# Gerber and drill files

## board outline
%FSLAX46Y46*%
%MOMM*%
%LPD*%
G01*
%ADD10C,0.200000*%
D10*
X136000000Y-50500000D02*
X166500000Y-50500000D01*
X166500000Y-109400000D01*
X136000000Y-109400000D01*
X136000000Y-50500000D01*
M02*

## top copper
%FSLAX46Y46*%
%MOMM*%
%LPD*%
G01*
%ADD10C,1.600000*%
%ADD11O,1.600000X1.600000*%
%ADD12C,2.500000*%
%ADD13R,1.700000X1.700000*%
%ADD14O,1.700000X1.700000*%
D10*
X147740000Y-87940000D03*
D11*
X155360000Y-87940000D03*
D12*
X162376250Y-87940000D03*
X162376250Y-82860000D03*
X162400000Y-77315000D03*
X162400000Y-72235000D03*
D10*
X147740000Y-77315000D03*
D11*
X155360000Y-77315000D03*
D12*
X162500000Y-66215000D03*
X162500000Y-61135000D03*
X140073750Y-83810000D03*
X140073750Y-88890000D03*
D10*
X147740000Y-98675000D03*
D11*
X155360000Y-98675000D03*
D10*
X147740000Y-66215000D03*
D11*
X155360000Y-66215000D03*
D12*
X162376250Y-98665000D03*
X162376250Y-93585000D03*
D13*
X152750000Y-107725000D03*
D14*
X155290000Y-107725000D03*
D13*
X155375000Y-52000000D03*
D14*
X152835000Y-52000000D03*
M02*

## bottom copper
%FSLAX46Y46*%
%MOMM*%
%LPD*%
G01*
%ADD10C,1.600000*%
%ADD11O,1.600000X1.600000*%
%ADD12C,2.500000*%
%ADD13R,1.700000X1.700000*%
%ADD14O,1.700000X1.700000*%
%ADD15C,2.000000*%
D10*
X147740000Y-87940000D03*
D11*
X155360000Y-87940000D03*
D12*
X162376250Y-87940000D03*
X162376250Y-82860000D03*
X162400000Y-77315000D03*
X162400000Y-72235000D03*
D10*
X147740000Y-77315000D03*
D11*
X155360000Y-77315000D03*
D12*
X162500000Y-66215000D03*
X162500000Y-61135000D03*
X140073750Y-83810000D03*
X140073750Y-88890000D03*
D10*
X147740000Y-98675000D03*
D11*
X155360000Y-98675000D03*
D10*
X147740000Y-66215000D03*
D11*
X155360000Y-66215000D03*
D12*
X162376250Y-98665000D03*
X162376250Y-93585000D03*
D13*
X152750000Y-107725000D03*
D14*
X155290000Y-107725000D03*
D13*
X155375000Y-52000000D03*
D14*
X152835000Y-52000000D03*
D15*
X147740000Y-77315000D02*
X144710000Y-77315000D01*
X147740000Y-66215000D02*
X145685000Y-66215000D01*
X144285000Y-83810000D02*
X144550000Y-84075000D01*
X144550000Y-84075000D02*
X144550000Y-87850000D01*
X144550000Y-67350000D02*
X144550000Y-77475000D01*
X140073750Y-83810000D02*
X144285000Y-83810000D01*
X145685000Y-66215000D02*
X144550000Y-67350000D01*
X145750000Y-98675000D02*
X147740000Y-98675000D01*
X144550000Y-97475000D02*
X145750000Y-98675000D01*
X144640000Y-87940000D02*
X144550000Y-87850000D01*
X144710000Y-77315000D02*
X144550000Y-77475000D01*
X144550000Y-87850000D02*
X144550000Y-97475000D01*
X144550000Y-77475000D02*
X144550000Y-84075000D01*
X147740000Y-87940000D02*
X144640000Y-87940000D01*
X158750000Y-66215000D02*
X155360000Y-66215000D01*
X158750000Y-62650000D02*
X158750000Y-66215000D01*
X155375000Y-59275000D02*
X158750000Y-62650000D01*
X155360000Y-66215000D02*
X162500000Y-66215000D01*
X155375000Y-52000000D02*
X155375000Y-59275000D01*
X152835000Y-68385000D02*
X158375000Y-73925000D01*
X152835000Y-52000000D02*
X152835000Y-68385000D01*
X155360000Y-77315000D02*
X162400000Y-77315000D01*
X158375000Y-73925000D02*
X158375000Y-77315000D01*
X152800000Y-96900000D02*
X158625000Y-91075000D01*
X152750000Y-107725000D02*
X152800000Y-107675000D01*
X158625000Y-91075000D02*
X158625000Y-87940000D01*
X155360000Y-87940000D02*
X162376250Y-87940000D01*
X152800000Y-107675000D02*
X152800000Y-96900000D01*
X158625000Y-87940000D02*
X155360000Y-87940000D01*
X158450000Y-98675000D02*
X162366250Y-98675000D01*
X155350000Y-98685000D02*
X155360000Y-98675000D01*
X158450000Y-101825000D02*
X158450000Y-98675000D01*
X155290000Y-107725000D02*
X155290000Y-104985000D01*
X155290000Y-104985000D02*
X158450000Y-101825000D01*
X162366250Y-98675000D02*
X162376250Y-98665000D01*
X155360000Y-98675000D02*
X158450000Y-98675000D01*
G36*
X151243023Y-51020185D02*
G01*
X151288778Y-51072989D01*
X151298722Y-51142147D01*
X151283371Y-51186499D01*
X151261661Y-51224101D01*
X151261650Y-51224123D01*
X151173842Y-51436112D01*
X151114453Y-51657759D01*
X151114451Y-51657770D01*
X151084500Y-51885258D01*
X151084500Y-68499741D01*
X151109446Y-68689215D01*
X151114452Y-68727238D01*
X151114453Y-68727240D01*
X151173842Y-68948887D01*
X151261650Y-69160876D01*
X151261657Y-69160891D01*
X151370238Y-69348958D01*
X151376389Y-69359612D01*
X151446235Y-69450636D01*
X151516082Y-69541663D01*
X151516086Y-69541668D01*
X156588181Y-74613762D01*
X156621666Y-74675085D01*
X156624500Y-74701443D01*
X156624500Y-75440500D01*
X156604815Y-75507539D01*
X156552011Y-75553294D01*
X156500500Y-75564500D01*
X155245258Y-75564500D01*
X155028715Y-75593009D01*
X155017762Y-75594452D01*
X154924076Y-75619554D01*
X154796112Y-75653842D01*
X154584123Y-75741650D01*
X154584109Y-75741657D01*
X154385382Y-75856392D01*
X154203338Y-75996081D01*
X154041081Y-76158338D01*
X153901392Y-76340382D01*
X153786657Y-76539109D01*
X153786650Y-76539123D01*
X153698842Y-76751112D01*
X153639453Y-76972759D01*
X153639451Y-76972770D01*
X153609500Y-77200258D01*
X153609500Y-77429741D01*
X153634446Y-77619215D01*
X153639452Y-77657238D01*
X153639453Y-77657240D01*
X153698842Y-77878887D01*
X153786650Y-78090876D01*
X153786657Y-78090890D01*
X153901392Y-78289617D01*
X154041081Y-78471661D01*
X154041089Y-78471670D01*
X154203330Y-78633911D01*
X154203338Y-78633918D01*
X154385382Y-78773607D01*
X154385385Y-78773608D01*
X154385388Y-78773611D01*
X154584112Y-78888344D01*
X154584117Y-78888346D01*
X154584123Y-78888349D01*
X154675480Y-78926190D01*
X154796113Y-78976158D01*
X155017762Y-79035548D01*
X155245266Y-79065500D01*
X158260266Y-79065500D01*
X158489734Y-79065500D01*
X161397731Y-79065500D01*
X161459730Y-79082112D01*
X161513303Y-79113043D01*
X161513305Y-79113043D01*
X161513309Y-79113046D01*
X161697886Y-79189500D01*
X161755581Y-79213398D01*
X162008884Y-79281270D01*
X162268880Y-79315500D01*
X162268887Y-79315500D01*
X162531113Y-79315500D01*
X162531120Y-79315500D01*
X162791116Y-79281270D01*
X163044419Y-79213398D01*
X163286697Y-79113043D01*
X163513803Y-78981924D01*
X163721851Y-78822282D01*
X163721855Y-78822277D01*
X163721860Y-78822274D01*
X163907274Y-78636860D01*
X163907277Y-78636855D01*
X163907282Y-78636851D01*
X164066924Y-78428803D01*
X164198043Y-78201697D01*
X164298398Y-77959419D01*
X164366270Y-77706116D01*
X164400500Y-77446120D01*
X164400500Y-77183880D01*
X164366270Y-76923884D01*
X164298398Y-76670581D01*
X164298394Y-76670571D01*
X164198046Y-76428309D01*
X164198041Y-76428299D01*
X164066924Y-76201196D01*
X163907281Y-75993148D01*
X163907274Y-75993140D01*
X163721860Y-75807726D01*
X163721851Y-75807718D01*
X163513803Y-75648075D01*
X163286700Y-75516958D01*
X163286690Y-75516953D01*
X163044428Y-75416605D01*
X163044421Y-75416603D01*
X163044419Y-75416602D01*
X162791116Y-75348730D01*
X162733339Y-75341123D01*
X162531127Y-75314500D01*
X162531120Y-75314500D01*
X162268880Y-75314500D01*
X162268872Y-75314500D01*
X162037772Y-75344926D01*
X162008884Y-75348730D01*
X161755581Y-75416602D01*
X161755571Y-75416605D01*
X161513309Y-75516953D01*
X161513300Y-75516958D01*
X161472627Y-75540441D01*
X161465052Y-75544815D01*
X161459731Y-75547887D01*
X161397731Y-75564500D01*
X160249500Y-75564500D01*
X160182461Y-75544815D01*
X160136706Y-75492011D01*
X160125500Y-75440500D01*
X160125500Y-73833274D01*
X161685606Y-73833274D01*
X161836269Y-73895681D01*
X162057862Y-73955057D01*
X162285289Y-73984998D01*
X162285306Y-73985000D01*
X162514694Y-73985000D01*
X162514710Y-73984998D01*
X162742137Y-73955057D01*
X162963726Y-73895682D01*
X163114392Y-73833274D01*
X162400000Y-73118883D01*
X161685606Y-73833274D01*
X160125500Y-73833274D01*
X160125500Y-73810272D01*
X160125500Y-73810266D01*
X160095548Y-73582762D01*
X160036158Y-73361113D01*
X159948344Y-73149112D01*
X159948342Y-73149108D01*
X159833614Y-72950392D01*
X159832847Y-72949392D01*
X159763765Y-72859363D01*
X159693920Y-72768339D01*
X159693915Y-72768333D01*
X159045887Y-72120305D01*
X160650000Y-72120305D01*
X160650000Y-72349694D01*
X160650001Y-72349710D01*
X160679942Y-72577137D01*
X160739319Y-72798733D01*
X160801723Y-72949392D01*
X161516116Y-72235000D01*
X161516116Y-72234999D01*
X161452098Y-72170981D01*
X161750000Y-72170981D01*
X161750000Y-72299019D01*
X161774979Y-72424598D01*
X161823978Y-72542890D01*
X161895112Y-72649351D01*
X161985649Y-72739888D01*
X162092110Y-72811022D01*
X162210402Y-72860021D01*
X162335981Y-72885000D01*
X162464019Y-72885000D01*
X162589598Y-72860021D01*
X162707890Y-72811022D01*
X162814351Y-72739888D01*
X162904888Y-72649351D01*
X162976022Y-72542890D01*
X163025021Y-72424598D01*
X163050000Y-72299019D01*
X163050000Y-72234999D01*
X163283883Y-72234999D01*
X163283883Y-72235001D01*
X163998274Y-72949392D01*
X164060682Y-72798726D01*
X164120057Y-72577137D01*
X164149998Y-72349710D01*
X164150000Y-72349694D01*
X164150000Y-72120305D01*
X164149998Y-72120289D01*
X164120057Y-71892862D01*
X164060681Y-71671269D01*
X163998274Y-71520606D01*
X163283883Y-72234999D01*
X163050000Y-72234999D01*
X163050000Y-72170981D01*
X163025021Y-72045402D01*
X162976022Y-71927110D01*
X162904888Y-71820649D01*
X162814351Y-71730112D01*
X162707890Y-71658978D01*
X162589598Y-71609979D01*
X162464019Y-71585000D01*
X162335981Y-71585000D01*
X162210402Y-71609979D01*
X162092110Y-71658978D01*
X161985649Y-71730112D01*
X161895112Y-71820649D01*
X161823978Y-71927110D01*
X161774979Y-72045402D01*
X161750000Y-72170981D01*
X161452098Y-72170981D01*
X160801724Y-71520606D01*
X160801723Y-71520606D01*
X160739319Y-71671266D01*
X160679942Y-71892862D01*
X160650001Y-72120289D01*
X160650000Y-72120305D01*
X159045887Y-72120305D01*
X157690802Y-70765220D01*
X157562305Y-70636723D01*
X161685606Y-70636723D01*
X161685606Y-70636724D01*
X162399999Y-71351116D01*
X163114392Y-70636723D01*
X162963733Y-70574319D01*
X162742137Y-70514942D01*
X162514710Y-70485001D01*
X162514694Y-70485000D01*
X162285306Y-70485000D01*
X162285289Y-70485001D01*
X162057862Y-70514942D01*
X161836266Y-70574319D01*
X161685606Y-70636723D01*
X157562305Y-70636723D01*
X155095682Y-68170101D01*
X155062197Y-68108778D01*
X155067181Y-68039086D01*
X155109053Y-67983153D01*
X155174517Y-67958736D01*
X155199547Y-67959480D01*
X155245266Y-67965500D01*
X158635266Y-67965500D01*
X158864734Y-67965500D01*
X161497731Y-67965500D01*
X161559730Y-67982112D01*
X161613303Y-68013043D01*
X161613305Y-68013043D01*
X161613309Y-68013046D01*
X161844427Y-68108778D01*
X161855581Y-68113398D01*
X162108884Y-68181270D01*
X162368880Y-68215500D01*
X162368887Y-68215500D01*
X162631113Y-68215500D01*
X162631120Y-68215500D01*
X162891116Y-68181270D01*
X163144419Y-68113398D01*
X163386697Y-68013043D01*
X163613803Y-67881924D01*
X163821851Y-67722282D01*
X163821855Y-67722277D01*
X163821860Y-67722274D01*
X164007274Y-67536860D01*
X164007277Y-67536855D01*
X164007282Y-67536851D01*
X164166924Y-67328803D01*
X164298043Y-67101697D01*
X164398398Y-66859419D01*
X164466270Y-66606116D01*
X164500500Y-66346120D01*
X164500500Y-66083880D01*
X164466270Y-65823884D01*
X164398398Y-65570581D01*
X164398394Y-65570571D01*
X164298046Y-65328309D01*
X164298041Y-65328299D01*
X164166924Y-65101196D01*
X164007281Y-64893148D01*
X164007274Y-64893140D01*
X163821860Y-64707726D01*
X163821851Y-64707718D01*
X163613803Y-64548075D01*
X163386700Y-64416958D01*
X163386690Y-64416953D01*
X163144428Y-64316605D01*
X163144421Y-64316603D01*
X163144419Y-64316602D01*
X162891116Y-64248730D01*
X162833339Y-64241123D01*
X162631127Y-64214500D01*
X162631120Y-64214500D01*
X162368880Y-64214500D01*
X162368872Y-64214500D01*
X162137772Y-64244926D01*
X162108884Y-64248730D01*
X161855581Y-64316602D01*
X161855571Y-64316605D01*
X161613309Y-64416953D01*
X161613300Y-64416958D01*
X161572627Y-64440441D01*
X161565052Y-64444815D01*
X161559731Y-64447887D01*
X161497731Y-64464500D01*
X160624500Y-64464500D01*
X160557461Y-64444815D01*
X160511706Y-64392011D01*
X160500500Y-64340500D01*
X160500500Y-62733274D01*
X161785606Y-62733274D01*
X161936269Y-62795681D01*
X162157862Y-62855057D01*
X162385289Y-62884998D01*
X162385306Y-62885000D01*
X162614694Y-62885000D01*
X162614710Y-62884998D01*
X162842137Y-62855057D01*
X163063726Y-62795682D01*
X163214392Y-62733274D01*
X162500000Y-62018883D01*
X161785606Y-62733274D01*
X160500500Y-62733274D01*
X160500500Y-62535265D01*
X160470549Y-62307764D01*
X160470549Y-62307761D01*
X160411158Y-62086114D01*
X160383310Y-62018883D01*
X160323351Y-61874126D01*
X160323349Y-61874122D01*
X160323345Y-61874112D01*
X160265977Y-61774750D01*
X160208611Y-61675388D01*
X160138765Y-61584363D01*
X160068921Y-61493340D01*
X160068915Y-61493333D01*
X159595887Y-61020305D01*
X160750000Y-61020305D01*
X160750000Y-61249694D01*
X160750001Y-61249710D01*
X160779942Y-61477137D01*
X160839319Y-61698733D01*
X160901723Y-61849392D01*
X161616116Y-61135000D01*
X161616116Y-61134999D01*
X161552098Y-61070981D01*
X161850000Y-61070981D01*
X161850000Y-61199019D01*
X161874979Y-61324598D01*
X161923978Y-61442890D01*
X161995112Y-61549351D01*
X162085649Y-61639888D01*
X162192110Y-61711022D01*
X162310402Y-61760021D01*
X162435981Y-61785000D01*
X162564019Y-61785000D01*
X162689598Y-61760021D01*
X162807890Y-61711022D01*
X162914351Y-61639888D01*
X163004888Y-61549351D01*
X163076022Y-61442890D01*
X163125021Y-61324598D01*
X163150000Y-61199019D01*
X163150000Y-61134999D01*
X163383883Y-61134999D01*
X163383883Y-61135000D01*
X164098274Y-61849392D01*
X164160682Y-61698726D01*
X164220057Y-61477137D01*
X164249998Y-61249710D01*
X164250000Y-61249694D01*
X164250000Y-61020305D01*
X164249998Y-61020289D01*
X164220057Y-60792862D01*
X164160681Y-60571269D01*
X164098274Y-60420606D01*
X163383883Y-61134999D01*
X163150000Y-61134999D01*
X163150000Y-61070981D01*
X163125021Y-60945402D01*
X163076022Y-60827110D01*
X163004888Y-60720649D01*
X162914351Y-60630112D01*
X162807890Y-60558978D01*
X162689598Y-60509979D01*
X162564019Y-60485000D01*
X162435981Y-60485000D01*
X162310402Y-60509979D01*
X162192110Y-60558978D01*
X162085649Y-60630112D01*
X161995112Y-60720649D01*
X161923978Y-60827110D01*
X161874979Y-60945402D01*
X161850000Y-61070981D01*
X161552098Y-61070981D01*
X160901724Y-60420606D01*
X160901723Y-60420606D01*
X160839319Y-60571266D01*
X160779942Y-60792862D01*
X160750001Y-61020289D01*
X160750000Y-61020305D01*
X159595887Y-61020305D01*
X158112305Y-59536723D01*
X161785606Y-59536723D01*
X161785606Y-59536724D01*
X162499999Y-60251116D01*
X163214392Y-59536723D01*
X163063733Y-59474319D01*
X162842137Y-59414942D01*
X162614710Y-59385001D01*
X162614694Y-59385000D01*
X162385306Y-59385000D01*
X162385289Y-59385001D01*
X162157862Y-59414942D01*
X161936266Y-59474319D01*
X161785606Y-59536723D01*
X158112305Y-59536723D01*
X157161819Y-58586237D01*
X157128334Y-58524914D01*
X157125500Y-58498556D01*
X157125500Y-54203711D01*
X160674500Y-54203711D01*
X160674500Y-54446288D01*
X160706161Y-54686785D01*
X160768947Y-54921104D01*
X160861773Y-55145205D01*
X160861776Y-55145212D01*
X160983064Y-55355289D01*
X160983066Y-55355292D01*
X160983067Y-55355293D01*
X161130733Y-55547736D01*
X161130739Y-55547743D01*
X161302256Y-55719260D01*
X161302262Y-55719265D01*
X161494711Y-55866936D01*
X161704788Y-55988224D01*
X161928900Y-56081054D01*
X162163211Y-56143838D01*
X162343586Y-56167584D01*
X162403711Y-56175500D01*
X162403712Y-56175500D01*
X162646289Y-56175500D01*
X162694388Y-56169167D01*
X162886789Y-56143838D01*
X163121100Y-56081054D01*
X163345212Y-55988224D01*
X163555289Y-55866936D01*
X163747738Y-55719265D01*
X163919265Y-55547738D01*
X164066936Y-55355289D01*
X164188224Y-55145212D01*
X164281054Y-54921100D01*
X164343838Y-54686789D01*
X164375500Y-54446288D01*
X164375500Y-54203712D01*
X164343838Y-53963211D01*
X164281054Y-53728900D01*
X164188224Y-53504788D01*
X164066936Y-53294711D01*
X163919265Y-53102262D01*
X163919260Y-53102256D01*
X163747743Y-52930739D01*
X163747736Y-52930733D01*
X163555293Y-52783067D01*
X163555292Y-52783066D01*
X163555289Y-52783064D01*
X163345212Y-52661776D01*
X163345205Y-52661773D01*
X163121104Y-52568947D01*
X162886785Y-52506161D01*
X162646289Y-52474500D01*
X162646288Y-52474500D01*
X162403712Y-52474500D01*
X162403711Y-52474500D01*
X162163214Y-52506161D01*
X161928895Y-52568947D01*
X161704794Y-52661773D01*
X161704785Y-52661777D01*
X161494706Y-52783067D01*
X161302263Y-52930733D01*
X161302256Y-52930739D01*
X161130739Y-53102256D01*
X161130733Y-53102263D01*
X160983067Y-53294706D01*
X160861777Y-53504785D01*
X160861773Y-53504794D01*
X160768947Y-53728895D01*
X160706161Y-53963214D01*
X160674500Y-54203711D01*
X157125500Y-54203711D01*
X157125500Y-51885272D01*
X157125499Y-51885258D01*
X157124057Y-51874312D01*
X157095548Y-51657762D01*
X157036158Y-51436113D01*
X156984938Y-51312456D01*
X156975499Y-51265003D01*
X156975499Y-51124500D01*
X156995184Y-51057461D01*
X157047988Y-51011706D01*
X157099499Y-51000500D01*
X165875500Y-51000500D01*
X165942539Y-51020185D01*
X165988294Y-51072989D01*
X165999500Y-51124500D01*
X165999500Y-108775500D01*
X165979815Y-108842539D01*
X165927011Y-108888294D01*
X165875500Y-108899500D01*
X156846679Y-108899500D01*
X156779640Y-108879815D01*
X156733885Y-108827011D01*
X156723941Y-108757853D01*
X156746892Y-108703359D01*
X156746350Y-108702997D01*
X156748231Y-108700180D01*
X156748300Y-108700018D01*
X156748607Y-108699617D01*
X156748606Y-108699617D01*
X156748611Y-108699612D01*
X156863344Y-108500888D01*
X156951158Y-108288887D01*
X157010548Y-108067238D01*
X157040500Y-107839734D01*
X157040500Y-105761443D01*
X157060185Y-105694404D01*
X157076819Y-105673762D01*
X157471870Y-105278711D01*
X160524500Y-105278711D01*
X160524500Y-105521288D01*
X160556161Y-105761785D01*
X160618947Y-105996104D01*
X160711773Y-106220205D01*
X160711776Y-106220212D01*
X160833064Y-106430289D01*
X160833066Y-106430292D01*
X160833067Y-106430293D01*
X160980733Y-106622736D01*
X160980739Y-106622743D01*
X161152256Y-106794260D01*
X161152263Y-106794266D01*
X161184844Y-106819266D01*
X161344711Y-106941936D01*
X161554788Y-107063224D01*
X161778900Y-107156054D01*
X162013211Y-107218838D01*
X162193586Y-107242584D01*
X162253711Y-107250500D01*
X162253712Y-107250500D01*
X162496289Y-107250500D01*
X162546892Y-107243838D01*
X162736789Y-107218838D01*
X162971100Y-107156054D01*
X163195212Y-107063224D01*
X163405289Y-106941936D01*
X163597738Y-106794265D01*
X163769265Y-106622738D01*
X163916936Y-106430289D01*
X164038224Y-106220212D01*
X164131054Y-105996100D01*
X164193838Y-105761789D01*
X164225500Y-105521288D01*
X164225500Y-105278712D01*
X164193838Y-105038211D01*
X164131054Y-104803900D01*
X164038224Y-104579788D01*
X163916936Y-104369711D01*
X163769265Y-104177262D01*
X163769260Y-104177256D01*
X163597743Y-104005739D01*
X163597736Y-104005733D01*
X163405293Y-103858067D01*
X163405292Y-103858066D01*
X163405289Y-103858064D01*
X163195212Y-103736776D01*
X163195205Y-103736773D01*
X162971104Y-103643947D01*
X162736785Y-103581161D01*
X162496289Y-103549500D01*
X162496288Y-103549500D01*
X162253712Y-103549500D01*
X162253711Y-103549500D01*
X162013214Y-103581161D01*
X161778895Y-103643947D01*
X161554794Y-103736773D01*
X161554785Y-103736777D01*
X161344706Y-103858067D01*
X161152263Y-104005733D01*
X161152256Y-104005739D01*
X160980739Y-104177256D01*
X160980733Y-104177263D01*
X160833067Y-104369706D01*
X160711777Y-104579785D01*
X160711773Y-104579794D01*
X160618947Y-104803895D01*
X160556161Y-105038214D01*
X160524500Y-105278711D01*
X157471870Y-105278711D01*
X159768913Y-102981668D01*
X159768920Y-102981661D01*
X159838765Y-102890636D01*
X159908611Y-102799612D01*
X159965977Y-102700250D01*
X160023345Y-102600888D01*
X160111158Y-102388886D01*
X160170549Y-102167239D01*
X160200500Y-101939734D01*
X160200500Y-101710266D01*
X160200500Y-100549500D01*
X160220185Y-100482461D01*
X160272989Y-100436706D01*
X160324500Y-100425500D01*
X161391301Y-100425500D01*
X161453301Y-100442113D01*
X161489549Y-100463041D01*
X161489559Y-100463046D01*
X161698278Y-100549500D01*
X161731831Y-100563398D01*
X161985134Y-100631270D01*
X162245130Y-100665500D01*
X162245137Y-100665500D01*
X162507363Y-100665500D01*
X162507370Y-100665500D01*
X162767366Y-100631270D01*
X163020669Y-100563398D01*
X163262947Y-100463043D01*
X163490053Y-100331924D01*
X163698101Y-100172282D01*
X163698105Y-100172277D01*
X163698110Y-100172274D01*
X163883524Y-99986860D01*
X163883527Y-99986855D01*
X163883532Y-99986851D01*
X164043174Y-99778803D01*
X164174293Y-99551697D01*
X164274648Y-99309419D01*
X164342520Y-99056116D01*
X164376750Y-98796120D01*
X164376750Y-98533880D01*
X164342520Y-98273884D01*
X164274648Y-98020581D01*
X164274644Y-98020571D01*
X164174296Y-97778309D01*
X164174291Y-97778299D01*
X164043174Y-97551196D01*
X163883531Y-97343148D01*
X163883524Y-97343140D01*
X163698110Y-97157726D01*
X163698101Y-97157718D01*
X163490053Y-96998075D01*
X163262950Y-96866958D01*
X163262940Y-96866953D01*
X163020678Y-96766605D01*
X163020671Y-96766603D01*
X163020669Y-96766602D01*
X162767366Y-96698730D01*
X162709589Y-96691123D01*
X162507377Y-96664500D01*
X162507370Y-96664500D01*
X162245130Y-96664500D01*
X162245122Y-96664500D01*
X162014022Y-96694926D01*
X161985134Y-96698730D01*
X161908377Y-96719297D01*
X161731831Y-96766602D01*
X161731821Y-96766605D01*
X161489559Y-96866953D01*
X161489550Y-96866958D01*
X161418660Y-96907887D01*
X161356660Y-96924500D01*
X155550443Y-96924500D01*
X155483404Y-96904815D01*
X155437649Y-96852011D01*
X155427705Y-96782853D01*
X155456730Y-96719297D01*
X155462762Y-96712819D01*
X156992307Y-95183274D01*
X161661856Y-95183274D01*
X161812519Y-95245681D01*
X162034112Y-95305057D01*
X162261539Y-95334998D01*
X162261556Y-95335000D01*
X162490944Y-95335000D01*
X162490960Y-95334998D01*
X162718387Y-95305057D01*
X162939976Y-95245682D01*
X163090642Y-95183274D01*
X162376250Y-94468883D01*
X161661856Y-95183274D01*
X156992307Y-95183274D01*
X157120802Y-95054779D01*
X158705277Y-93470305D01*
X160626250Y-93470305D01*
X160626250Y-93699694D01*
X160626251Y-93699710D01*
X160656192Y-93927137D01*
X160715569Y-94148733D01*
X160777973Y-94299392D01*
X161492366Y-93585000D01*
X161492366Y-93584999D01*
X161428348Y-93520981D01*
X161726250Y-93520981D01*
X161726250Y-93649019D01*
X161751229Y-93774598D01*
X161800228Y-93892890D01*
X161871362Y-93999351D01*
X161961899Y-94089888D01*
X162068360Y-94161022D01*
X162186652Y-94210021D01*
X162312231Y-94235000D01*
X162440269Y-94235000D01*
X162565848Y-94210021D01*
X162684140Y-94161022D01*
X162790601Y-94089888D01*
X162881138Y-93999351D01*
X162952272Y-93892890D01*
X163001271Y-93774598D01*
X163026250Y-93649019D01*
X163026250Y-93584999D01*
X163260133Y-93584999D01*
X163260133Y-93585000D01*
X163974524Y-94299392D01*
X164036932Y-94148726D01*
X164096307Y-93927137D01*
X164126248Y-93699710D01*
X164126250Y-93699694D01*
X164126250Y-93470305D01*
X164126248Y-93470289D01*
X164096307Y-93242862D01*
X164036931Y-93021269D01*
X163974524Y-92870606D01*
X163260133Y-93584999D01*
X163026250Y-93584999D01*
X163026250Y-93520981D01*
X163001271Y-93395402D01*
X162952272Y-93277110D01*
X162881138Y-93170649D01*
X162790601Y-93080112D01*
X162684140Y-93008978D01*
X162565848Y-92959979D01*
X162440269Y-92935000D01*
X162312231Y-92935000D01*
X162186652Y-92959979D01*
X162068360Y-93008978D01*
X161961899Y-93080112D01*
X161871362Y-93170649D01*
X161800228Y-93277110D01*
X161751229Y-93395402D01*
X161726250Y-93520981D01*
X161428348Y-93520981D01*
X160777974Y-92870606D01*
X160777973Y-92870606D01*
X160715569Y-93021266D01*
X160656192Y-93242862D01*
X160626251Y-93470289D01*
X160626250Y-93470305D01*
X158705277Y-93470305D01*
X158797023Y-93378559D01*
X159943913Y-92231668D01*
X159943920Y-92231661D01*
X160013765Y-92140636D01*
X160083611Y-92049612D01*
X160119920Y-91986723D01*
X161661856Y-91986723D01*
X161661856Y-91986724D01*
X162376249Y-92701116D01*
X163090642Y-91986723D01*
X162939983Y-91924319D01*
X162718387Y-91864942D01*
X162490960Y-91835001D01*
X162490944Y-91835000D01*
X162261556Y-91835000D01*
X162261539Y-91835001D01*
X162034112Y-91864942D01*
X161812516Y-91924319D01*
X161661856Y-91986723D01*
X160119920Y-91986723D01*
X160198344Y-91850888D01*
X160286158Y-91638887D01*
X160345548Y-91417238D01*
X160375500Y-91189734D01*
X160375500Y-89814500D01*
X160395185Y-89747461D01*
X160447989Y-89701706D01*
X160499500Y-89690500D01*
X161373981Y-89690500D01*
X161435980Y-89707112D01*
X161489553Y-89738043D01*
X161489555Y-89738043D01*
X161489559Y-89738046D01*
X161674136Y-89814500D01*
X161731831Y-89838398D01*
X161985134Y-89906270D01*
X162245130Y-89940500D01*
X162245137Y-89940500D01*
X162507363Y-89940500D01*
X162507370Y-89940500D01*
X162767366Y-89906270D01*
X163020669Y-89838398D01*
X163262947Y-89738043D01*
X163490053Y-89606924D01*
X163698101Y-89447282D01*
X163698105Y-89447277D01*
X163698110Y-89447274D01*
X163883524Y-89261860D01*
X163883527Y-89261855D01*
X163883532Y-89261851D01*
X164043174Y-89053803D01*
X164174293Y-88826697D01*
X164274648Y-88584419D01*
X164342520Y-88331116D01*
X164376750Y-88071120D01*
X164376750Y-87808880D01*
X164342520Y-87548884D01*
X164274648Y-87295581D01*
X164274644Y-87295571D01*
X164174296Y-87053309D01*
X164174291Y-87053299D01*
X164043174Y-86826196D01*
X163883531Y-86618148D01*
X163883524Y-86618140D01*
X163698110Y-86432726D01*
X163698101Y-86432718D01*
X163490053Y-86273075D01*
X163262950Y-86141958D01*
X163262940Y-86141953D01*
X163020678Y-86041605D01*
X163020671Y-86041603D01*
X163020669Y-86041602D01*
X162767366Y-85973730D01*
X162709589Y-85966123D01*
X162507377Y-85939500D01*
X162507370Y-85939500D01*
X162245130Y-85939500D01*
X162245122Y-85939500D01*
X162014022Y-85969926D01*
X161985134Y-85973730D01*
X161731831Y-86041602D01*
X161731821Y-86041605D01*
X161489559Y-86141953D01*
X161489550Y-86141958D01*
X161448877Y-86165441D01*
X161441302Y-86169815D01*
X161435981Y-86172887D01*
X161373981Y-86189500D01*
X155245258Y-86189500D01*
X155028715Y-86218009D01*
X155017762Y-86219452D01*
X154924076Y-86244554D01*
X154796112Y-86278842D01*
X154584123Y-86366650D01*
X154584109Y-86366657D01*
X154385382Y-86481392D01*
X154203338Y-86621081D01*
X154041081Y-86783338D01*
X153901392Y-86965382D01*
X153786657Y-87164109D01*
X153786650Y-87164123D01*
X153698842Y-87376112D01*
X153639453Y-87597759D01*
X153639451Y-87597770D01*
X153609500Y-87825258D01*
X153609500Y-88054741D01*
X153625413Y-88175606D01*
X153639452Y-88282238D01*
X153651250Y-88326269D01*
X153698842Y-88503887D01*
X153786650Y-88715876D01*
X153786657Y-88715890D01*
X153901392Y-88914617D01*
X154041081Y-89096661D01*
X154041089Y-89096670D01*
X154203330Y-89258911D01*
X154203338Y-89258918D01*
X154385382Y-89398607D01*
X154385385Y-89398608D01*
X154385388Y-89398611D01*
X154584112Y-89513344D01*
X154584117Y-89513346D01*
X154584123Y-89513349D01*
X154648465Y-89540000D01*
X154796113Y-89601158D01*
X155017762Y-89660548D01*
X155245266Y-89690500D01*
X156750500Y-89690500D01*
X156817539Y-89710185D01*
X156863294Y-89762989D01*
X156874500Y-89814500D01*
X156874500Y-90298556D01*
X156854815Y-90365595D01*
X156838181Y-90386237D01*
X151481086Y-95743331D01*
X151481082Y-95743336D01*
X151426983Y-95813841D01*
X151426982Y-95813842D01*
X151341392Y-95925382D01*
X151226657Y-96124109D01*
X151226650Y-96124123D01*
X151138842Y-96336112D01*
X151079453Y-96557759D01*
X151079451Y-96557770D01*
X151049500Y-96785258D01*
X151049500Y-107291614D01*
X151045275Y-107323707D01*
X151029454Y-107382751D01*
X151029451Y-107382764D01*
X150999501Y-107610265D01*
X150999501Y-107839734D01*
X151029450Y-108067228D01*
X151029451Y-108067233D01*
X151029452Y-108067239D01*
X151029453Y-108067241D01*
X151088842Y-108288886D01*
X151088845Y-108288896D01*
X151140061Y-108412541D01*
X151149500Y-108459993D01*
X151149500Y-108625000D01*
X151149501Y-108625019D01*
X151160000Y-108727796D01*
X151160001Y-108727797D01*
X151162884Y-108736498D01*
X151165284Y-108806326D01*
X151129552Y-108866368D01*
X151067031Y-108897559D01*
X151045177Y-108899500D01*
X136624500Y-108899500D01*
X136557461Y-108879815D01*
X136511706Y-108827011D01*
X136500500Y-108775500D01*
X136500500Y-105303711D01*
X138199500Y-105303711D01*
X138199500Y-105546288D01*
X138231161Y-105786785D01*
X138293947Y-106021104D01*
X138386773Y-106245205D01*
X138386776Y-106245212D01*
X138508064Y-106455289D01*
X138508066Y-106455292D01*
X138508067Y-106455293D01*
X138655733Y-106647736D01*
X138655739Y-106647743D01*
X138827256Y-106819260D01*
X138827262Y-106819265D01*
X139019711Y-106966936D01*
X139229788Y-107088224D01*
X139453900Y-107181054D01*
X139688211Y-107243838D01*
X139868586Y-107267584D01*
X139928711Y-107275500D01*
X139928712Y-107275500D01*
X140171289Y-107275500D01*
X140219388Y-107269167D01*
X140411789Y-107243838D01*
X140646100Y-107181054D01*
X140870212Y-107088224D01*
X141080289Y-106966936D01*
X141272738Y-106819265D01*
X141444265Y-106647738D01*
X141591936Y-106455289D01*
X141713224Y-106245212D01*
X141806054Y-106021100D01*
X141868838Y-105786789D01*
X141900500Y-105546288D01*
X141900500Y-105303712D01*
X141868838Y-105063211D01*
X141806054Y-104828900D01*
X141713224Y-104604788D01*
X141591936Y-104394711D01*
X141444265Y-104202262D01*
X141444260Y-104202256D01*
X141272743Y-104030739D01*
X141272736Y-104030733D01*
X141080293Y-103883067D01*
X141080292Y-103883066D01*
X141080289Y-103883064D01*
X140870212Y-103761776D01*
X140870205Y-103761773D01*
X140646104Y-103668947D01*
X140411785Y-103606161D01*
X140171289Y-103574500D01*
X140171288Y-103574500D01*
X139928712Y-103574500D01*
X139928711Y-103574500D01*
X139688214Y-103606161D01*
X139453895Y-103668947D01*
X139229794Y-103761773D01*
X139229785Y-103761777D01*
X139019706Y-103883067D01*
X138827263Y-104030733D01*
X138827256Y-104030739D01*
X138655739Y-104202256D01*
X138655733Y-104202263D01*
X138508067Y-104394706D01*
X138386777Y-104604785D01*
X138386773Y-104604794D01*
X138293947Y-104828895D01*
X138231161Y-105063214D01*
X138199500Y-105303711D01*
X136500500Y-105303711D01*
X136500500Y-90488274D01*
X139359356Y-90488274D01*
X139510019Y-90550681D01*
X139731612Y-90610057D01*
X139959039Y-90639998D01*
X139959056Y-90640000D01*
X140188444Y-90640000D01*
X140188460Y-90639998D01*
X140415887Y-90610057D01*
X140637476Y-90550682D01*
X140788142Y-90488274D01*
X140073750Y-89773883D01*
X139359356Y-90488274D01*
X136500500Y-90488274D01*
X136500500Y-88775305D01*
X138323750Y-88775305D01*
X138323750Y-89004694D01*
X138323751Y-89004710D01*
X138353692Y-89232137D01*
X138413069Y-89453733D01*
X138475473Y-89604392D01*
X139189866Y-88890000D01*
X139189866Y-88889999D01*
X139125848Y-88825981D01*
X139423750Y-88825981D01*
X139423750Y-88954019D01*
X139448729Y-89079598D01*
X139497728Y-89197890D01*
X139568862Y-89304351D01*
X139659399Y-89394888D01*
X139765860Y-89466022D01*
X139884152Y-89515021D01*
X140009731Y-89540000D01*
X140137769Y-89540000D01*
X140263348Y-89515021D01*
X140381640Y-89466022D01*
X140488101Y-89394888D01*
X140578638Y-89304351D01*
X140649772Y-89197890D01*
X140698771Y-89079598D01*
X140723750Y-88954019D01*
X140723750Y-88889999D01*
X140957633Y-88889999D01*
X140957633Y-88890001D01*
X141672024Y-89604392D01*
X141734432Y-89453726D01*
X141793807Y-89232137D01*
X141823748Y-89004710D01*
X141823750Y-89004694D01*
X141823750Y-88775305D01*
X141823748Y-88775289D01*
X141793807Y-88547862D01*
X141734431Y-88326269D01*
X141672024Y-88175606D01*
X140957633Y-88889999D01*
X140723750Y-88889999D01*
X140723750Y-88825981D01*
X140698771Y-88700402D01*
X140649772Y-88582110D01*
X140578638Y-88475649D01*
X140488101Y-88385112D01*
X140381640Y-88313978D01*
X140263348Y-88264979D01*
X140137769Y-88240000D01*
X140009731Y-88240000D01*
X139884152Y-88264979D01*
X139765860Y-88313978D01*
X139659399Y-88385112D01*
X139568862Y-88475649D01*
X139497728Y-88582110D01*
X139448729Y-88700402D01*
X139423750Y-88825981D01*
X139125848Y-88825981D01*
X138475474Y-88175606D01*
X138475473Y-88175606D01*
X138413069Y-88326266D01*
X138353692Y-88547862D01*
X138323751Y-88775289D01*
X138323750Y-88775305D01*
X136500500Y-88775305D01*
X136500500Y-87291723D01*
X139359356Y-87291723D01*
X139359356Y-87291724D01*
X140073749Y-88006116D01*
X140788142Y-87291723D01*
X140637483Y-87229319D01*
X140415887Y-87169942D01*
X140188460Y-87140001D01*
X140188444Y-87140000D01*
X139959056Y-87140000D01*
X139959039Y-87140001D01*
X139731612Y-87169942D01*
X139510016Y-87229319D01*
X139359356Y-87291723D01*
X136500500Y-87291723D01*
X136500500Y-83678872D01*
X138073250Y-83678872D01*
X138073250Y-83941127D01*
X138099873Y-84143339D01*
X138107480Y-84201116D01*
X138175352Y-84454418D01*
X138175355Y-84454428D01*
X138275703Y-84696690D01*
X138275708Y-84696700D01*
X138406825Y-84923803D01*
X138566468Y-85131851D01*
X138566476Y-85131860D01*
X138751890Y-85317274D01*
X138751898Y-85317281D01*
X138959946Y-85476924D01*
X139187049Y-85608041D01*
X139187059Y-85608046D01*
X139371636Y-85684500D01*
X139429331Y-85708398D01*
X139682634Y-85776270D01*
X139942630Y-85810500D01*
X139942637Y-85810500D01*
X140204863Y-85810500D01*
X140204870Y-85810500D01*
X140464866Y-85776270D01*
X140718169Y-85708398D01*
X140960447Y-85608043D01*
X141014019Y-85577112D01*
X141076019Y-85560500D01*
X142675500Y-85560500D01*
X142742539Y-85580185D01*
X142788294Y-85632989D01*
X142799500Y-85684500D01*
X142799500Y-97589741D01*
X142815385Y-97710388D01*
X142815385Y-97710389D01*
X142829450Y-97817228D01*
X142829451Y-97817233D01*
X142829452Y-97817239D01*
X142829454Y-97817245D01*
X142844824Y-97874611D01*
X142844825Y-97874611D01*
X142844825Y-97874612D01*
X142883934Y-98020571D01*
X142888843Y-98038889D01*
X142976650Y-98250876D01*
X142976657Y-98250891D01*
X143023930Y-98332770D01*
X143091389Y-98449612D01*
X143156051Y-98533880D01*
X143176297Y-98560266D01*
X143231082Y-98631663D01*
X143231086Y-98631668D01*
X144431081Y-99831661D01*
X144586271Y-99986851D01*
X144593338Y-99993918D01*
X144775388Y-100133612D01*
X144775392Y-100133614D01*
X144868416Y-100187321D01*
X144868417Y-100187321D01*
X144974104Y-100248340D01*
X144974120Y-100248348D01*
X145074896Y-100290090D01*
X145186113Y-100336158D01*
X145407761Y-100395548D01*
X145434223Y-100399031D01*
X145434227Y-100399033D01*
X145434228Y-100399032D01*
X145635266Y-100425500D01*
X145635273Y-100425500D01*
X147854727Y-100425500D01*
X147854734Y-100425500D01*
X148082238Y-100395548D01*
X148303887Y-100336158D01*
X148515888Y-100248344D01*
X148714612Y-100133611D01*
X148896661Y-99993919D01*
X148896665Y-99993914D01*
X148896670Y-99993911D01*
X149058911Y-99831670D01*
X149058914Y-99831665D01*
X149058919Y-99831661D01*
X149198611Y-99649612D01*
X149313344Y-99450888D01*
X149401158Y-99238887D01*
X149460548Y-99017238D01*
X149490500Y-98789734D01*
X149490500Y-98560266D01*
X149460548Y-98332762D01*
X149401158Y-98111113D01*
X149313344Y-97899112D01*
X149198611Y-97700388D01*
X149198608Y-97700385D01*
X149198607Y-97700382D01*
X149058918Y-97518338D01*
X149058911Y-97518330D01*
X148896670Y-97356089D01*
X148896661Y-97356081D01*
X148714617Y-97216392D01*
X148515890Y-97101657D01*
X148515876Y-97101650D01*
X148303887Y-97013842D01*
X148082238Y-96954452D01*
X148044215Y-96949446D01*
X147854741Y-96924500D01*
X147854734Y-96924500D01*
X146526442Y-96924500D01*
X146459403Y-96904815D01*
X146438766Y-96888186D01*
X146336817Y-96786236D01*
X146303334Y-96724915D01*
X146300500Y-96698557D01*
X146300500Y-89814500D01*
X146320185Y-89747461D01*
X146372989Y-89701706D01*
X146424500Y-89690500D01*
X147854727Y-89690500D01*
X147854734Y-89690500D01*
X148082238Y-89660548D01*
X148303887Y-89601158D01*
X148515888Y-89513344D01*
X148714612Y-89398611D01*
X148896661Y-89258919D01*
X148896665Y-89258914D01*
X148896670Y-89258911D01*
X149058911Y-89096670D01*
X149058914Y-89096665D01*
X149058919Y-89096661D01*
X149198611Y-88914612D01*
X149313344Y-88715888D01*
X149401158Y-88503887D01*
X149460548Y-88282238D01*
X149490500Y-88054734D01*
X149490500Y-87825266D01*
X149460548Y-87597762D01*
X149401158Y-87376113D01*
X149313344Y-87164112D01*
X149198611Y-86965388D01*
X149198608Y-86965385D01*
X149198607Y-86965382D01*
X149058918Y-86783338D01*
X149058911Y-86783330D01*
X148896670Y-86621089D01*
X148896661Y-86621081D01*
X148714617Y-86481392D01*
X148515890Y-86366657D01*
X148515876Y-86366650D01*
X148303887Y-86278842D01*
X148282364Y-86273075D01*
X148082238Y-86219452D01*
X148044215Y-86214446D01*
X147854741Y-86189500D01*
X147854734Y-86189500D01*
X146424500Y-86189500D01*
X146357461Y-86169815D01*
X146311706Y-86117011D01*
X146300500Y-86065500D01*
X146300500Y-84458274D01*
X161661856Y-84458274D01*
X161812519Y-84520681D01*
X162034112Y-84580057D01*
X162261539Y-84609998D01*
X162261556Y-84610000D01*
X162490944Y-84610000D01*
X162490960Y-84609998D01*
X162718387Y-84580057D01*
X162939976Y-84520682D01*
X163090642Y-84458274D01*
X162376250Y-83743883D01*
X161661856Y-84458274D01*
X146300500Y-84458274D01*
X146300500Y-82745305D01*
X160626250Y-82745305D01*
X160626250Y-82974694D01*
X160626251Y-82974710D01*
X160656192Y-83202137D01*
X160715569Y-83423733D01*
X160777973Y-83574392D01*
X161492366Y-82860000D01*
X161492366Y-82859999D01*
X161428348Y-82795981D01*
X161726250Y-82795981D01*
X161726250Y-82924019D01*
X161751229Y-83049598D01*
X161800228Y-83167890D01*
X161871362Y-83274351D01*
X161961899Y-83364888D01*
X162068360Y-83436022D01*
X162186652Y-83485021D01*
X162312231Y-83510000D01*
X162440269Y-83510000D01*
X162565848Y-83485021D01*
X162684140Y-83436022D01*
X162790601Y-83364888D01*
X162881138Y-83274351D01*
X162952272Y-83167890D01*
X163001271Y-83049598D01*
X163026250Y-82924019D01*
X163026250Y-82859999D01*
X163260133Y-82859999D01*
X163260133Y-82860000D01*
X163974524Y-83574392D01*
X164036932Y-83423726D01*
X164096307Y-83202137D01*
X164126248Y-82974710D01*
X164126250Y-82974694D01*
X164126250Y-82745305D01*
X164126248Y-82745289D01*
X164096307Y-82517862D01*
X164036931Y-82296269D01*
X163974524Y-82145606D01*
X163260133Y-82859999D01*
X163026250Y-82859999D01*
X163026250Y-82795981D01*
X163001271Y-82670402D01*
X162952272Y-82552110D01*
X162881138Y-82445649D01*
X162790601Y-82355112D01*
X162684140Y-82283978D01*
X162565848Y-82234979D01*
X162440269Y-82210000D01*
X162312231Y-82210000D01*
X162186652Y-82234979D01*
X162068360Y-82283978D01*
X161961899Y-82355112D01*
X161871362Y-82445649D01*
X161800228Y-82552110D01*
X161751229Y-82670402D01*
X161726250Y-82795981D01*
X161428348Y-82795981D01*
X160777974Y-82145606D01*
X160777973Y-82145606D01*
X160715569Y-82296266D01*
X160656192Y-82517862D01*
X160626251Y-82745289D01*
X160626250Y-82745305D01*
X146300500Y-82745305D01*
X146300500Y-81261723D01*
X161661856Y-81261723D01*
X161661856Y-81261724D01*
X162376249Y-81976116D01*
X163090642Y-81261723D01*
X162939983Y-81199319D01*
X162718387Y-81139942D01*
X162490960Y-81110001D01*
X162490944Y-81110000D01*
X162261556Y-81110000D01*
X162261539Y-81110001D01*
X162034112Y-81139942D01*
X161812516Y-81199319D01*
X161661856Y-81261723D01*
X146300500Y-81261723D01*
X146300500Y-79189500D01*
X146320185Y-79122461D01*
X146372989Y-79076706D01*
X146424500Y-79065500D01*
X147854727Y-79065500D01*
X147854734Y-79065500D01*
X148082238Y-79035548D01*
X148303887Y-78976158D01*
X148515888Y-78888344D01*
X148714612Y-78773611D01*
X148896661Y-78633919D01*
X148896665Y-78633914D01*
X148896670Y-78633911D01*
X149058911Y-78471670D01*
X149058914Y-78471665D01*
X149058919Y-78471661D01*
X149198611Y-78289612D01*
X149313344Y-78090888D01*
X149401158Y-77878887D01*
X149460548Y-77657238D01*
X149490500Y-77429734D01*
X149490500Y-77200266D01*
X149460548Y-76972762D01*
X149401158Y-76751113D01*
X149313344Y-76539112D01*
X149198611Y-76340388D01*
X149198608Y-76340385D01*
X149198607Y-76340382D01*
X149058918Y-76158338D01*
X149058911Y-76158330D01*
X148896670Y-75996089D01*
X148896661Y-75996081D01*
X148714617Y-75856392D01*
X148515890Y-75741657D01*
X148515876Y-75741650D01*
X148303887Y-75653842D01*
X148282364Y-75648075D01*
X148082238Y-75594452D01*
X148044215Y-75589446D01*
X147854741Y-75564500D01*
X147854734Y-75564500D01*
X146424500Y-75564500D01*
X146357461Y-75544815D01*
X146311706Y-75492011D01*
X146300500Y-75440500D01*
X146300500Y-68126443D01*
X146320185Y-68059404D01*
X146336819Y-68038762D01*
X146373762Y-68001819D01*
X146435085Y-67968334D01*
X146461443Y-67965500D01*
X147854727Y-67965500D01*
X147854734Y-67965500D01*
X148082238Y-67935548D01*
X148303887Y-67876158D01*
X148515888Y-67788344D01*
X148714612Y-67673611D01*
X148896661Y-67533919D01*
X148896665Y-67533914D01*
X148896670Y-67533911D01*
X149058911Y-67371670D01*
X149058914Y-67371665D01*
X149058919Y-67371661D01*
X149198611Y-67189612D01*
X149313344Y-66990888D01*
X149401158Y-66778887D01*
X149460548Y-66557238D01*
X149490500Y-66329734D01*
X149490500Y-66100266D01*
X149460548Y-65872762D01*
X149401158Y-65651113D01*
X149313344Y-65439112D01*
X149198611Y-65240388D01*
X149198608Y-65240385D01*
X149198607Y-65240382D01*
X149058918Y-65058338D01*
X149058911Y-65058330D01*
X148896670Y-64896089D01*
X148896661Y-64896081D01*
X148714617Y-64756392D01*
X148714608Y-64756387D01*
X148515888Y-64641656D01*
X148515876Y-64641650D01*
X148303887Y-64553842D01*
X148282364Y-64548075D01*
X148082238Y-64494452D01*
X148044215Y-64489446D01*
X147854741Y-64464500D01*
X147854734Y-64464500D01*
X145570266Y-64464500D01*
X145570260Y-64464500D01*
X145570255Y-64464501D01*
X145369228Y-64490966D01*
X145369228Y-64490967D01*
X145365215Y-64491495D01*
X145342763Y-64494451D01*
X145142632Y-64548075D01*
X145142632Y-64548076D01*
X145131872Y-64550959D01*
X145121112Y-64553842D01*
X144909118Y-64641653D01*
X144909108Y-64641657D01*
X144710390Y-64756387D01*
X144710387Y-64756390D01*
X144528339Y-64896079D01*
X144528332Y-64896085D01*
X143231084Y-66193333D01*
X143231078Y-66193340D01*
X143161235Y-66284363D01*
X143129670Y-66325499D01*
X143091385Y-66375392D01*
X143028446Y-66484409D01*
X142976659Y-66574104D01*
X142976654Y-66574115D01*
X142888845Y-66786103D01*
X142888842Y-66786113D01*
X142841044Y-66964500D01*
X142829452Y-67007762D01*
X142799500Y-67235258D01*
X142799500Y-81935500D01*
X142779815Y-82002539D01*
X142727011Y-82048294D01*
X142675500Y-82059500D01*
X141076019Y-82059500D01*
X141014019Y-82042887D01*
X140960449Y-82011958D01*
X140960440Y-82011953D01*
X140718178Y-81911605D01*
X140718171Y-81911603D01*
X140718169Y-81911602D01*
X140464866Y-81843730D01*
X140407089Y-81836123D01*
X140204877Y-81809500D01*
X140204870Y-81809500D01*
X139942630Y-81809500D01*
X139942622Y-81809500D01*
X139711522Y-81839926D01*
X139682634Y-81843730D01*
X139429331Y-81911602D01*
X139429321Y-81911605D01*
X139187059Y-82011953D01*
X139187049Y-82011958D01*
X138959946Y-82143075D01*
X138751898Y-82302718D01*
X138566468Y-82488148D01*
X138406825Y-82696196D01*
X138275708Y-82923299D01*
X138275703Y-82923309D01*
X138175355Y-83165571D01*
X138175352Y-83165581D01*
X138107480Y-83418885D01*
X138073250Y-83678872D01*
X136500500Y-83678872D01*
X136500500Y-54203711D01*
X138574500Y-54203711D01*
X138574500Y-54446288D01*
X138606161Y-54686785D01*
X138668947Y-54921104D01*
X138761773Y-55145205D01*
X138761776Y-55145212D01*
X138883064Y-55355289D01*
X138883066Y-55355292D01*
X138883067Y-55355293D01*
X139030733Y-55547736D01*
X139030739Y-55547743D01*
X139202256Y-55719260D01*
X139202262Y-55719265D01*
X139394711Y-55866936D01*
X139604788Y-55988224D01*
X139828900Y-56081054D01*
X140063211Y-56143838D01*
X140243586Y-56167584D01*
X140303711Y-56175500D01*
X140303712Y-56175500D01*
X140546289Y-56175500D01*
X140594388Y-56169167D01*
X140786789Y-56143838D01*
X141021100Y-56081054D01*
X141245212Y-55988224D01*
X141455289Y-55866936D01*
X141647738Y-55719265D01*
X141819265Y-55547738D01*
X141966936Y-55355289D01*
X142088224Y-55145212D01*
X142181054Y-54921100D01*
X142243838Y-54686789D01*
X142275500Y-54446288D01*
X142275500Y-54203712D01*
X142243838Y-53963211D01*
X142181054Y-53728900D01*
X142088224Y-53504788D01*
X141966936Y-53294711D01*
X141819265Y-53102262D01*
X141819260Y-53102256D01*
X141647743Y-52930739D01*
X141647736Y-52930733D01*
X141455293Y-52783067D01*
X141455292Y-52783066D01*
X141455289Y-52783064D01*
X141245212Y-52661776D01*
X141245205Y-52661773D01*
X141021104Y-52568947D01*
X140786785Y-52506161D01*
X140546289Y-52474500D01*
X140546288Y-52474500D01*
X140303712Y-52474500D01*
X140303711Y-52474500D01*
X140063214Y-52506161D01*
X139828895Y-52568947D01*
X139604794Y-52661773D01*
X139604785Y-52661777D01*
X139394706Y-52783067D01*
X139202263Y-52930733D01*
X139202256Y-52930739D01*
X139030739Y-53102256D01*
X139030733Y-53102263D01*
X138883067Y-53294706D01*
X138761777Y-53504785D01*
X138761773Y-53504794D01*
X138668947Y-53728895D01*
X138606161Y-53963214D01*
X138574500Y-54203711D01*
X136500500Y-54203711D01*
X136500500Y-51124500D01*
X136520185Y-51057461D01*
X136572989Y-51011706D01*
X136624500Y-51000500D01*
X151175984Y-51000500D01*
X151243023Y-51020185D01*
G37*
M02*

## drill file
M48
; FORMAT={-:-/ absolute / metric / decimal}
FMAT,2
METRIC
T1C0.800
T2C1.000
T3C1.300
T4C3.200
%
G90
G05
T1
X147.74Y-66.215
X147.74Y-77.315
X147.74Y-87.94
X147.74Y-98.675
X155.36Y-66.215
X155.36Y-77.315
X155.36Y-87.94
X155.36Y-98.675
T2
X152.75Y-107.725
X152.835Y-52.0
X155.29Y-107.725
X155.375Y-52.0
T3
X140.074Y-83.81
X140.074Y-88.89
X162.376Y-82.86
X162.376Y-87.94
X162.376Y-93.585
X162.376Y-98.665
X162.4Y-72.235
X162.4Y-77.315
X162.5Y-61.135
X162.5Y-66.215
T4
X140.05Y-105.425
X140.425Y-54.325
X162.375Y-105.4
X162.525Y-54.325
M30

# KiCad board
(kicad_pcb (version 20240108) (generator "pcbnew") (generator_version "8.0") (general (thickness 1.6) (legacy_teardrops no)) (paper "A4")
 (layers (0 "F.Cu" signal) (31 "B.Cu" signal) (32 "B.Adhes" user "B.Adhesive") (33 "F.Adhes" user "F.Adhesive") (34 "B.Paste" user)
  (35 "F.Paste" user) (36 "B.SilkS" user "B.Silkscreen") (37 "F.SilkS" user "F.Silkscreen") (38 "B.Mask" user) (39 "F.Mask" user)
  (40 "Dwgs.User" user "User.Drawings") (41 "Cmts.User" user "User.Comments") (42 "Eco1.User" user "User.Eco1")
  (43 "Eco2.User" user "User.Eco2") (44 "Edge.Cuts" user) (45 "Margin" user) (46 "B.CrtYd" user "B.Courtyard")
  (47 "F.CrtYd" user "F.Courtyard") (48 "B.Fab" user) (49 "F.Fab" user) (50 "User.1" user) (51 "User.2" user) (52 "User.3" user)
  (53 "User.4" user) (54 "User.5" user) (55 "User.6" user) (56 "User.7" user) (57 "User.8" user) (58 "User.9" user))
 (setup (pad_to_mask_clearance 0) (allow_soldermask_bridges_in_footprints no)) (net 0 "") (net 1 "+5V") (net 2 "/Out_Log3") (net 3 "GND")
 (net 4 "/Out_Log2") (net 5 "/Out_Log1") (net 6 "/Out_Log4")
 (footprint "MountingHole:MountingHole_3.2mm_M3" (layer "F.Cu") (at 140.425 54.325)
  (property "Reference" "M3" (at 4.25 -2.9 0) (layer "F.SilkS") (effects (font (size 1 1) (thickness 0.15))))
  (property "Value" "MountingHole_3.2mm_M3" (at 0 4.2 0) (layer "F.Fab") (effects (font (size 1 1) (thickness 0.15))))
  (pad "" np_thru_hole circle (at 0 0) (size 3.2 3.2) (drill 3.2) (layers "*.Cu" "*.Mask")))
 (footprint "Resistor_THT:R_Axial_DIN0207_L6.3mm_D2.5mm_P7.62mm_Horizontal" (layer "F.Cu") (at 147.74 87.94)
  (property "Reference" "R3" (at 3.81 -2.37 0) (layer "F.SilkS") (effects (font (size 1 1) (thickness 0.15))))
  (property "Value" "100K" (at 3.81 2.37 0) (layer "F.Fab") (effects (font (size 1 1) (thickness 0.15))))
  (pad "1" thru_hole circle (at 0 0) (size 1.6 1.6) (drill 0.8) (layers "*.Cu" "*.Mask") (remove_unused_layers no) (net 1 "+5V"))
  (pad "2" thru_hole oval (at 7.62 0) (size 1.6 1.6) (drill 0.8) (layers "*.Cu" "*.Mask") (remove_unused_layers no) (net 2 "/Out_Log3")))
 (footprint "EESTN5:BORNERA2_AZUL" (layer "F.Cu") (at 162.37625 85.4 90)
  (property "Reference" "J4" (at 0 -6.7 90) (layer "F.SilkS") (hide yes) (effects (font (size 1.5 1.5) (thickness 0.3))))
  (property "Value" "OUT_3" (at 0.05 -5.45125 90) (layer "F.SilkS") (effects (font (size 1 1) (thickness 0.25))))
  (pad "1" thru_hole circle (at -2.54 0 90) (size 2.5 2.5) (drill 1.3) (layers "*.Cu" "*.Mask" "F.SilkS") (remove_unused_layers no)
   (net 2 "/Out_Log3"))
  (pad "2" thru_hole circle (at 2.54 0 90) (size 2.5 2.5) (drill 1.3) (layers "*.Cu" "*.Mask" "F.SilkS") (remove_unused_layers no)
   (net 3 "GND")))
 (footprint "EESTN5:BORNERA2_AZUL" (layer "F.Cu") (at 162.4 74.775 90)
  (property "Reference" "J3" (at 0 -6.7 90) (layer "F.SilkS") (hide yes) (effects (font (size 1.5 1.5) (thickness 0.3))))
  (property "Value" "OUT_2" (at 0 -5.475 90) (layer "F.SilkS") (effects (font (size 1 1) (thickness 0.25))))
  (pad "1" thru_hole circle (at -2.54 0 90) (size 2.5 2.5) (drill 1.3) (layers "*.Cu" "*.Mask" "F.SilkS") (remove_unused_layers no)
   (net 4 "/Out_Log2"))
  (pad "2" thru_hole circle (at 2.54 0 90) (size 2.5 2.5) (drill 1.3) (layers "*.Cu" "*.Mask" "F.SilkS") (remove_unused_layers no)
   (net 3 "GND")))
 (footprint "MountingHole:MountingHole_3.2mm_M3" (layer "F.Cu") (at 162.525 54.325)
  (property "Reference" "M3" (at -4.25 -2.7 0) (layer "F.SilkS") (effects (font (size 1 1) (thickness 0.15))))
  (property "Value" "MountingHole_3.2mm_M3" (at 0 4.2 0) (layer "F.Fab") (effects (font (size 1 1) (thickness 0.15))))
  (pad "" np_thru_hole circle (at 0 0) (size 3.2 3.2) (drill 3.2) (layers "*.Cu" "*.Mask")))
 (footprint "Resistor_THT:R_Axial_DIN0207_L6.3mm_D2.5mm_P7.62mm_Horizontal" (layer "F.Cu") (at 147.74 77.315)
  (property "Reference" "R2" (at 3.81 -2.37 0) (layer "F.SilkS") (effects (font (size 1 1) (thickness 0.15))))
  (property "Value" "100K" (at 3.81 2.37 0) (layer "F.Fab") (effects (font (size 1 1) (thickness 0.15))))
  (pad "1" thru_hole circle (at 0 0) (size 1.6 1.6) (drill 0.8) (layers "*.Cu" "*.Mask") (remove_unused_layers no) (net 1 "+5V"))
  (pad "2" thru_hole oval (at 7.62 0) (size 1.6 1.6) (drill 0.8) (layers "*.Cu" "*.Mask") (remove_unused_layers no) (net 4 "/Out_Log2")))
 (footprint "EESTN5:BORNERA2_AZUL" (layer "F.Cu") (at 162.5 63.675 90)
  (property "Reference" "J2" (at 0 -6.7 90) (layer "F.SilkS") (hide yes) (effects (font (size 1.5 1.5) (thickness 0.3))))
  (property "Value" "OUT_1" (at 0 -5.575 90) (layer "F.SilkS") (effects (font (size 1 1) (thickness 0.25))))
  (pad "1" thru_hole circle (at -2.54 0 90) (size 2.5 2.5) (drill 1.3) (layers "*.Cu" "*.Mask" "F.SilkS") (remove_unused_layers no)
   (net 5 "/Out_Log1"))
  (pad "2" thru_hole circle (at 2.54 0 90) (size 2.5 2.5) (drill 1.3) (layers "*.Cu" "*.Mask" "F.SilkS") (remove_unused_layers no)
   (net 3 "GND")))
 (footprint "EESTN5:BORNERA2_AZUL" (layer "F.Cu") (at 140.07375 86.35 -90)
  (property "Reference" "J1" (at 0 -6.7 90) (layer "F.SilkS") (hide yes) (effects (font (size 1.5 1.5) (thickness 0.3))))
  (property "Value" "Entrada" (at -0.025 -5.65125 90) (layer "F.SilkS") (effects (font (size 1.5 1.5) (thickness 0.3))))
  (pad "1" thru_hole circle (at -2.54 0 270) (size 2.5 2.5) (drill 1.3) (layers "*.Cu" "*.Mask" "F.SilkS") (remove_unused_layers no)
   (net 1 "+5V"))
  (pad "2" thru_hole circle (at 2.54 0 270) (size 2.5 2.5) (drill 1.3) (layers "*.Cu" "*.Mask" "F.SilkS") (remove_unused_layers no)
   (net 3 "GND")))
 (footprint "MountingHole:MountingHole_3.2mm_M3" (layer "F.Cu") (at 162.375 105.4)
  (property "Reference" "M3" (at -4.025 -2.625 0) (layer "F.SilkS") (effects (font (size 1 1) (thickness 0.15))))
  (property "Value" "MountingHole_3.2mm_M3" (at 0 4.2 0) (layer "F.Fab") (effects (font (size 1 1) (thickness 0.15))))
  (pad "" np_thru_hole circle (at 0 0) (size 3.2 3.2) (drill 3.2) (layers "*.Cu" "*.Mask")))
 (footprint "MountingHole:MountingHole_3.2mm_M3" (layer "F.Cu") (at 140.05 105.425)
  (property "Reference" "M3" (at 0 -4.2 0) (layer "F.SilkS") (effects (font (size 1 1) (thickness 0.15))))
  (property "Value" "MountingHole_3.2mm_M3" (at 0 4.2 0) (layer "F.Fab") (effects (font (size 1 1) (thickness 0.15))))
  (pad "" np_thru_hole circle (at 0 0) (size 3.2 3.2) (drill 3.2) (layers "*.Cu" "*.Mask")))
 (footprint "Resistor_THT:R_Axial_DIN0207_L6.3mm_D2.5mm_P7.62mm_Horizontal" (layer "F.Cu") (at 147.74 98.675)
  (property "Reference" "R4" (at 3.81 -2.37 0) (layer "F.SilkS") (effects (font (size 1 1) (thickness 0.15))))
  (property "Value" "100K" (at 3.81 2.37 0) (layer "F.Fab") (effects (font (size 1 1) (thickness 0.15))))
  (pad "1" thru_hole circle (at 0 0) (size 1.6 1.6) (drill 0.8) (layers "*.Cu" "*.Mask") (remove_unused_layers no) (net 1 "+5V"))
  (pad "2" thru_hole oval (at 7.62 0) (size 1.6 1.6) (drill 0.8) (layers "*.Cu" "*.Mask") (remove_unused_layers no) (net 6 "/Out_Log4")))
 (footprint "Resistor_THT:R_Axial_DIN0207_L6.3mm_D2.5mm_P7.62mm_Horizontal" (layer "F.Cu") (at 147.74 66.215)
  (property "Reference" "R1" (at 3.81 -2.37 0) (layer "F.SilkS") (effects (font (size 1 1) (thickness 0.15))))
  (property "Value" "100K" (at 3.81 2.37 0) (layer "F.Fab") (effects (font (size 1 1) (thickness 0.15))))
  (pad "1" thru_hole circle (at 0 0) (size 1.6 1.6) (drill 0.8) (layers "*.Cu" "*.Mask") (remove_unused_layers no) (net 1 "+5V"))
  (pad "2" thru_hole oval (at 7.62 0) (size 1.6 1.6) (drill 0.8) (layers "*.Cu" "*.Mask") (remove_unused_layers no) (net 5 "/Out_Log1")))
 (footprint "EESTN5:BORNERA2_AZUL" (layer "F.Cu") (at 162.37625 96.125 90)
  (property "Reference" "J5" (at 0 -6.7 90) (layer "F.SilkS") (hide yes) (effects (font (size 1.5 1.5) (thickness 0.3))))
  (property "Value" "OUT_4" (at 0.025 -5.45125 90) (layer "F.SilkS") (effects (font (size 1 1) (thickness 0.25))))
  (pad "1" thru_hole circle (at -2.54 0 90) (size 2.5 2.5) (drill 1.3) (layers "*.Cu" "*.Mask" "F.SilkS") (remove_unused_layers no)
   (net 6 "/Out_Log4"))
  (pad "2" thru_hole circle (at 2.54 0 90) (size 2.5 2.5) (drill 1.3) (layers "*.Cu" "*.Mask" "F.SilkS") (remove_unused_layers no)
   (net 3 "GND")))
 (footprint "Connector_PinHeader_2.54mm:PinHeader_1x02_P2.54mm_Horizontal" (layer "B.Cu") (at 152.75 107.725 -90)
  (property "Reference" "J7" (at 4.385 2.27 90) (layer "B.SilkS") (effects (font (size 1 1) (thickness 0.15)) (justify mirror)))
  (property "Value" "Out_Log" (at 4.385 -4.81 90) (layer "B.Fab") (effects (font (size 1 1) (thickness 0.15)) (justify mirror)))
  (pad "1" thru_hole rect (at 0 0 270) (size 1.7 1.7) (drill 1) (layers "*.Cu" "*.Mask") (remove_unused_layers no) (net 2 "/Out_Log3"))
  (pad "2" thru_hole oval (at 0 -2.54 270) (size 1.7 1.7) (drill 1) (layers "*.Cu" "*.Mask") (remove_unused_layers no) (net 6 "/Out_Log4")))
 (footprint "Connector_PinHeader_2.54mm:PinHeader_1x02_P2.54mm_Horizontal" (layer "B.Cu") (at 155.375 52 90)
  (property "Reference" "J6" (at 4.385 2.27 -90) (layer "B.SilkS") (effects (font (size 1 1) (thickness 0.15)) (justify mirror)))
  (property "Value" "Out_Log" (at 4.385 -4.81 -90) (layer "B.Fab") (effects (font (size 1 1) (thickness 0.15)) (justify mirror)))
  (pad "1" thru_hole rect (at 0 0 90) (size 1.7 1.7) (drill 1) (layers "*.Cu" "*.Mask") (remove_unused_layers no) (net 5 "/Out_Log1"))
  (pad "2" thru_hole oval (at 0 -2.54 90) (size 1.7 1.7) (drill 1) (layers "*.Cu" "*.Mask") (remove_unused_layers no) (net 4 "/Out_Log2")))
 (gr_rect (start 136 50.5) (end 166.5 109.4) (stroke (width 0.2) (type default)) (fill none) (layer "Edge.Cuts"))
 (segment (start 147.74 77.315) (end 144.71 77.315) (width 2) (layer "B.Cu") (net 1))
 (segment (start 147.74 66.215) (end 145.685 66.215) (width 2) (layer "B.Cu") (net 1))
 (segment (start 144.285 83.81) (end 144.55 84.075) (width 2) (layer "B.Cu") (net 1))
 (segment (start 144.55 84.075) (end 144.55 87.85) (width 2) (layer "B.Cu") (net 1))
 (segment (start 144.55 67.35) (end 144.55 77.475) (width 2) (layer "B.Cu") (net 1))
 (segment (start 140.07375 83.81) (end 144.285 83.81) (width 2) (layer "B.Cu") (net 1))
 (segment (start 145.685 66.215) (end 144.55 67.35) (width 2) (layer "B.Cu") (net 1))
 (segment (start 145.75 98.675) (end 147.74 98.675) (width 2) (layer "B.Cu") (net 1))
 (segment (start 144.55 97.475) (end 145.75 98.675) (width 2) (layer "B.Cu") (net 1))
 (segment (start 144.64 87.94) (end 144.55 87.85) (width 2) (layer "B.Cu") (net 1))
 (segment (start 144.71 77.315) (end 144.55 77.475) (width 2) (layer "B.Cu") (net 1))
 (segment (start 144.55 87.85) (end 144.55 97.475) (width 2) (layer "B.Cu") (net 1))
 (segment (start 144.55 77.475) (end 144.55 84.075) (width 2) (layer "B.Cu") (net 1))
 (segment (start 147.74 87.94) (end 144.64 87.94) (width 2) (layer "B.Cu") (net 1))
 (segment (start 158.75 66.215) (end 155.36 66.215) (width 2) (layer "B.Cu") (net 5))
 (segment (start 158.75 62.65) (end 158.75 66.215) (width 2) (layer "B.Cu") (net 5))
 (segment (start 155.375 59.275) (end 158.75 62.65) (width 2) (layer "B.Cu") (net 5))
 (segment (start 155.36 66.215) (end 162.5 66.215) (width 2) (layer "B.Cu") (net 5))
 (segment (start 155.375 52) (end 155.375 59.275) (width 2) (layer "B.Cu") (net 5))
 (segment (start 152.835 68.385) (end 158.375 73.925) (width 2) (layer "B.Cu") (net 4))
 (segment (start 152.835 52) (end 152.835 68.385) (width 2) (layer "B.Cu") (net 4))
 (segment (start 155.36 77.315) (end 162.4 77.315) (width 2) (layer "B.Cu") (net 4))
 (segment (start 158.375 73.925) (end 158.375 77.315) (width 2) (layer "B.Cu") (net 4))
 (segment (start 152.8 96.9) (end 158.625 91.075) (width 2) (layer "B.Cu") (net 2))
 (segment (start 152.75 107.725) (end 152.8 107.675) (width 2) (layer "B.Cu") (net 2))
 (segment (start 158.625 91.075) (end 158.625 87.94) (width 2) (layer "B.Cu") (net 2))
 (segment (start 155.36 87.94) (end 162.37625 87.94) (width 2) (layer "B.Cu") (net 2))
 (segment (start 152.8 107.675) (end 152.8 96.9) (width 2) (layer "B.Cu") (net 2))
 (segment (start 158.625 87.94) (end 155.36 87.94) (width 2) (layer "B.Cu") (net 2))
 (segment (start 158.45 98.675) (end 162.36625 98.675) (width 2) (layer "B.Cu") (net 6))
 (segment (start 155.35 98.685) (end 155.36 98.675) (width 2) (layer "B.Cu") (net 6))
 (segment (start 158.45 101.825) (end 158.45 98.675) (width 2) (layer "B.Cu") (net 6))
 (segment (start 155.29 107.725) (end 155.29 104.985) (width 2) (layer "B.Cu") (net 6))
 (segment (start 155.29 104.985) (end 158.45 101.825) (width 2) (layer "B.Cu") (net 6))
 (segment (start 162.36625 98.675) (end 162.37625 98.665) (width 2) (layer "B.Cu") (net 6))
 (segment (start 155.36 98.675) (end 158.45 98.675) (width 2) (layer "B.Cu") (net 6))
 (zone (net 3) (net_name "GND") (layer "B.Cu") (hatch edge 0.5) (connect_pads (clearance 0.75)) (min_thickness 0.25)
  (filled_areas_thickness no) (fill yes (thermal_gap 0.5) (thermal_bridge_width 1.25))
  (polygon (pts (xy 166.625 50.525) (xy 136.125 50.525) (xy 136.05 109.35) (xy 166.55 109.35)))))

